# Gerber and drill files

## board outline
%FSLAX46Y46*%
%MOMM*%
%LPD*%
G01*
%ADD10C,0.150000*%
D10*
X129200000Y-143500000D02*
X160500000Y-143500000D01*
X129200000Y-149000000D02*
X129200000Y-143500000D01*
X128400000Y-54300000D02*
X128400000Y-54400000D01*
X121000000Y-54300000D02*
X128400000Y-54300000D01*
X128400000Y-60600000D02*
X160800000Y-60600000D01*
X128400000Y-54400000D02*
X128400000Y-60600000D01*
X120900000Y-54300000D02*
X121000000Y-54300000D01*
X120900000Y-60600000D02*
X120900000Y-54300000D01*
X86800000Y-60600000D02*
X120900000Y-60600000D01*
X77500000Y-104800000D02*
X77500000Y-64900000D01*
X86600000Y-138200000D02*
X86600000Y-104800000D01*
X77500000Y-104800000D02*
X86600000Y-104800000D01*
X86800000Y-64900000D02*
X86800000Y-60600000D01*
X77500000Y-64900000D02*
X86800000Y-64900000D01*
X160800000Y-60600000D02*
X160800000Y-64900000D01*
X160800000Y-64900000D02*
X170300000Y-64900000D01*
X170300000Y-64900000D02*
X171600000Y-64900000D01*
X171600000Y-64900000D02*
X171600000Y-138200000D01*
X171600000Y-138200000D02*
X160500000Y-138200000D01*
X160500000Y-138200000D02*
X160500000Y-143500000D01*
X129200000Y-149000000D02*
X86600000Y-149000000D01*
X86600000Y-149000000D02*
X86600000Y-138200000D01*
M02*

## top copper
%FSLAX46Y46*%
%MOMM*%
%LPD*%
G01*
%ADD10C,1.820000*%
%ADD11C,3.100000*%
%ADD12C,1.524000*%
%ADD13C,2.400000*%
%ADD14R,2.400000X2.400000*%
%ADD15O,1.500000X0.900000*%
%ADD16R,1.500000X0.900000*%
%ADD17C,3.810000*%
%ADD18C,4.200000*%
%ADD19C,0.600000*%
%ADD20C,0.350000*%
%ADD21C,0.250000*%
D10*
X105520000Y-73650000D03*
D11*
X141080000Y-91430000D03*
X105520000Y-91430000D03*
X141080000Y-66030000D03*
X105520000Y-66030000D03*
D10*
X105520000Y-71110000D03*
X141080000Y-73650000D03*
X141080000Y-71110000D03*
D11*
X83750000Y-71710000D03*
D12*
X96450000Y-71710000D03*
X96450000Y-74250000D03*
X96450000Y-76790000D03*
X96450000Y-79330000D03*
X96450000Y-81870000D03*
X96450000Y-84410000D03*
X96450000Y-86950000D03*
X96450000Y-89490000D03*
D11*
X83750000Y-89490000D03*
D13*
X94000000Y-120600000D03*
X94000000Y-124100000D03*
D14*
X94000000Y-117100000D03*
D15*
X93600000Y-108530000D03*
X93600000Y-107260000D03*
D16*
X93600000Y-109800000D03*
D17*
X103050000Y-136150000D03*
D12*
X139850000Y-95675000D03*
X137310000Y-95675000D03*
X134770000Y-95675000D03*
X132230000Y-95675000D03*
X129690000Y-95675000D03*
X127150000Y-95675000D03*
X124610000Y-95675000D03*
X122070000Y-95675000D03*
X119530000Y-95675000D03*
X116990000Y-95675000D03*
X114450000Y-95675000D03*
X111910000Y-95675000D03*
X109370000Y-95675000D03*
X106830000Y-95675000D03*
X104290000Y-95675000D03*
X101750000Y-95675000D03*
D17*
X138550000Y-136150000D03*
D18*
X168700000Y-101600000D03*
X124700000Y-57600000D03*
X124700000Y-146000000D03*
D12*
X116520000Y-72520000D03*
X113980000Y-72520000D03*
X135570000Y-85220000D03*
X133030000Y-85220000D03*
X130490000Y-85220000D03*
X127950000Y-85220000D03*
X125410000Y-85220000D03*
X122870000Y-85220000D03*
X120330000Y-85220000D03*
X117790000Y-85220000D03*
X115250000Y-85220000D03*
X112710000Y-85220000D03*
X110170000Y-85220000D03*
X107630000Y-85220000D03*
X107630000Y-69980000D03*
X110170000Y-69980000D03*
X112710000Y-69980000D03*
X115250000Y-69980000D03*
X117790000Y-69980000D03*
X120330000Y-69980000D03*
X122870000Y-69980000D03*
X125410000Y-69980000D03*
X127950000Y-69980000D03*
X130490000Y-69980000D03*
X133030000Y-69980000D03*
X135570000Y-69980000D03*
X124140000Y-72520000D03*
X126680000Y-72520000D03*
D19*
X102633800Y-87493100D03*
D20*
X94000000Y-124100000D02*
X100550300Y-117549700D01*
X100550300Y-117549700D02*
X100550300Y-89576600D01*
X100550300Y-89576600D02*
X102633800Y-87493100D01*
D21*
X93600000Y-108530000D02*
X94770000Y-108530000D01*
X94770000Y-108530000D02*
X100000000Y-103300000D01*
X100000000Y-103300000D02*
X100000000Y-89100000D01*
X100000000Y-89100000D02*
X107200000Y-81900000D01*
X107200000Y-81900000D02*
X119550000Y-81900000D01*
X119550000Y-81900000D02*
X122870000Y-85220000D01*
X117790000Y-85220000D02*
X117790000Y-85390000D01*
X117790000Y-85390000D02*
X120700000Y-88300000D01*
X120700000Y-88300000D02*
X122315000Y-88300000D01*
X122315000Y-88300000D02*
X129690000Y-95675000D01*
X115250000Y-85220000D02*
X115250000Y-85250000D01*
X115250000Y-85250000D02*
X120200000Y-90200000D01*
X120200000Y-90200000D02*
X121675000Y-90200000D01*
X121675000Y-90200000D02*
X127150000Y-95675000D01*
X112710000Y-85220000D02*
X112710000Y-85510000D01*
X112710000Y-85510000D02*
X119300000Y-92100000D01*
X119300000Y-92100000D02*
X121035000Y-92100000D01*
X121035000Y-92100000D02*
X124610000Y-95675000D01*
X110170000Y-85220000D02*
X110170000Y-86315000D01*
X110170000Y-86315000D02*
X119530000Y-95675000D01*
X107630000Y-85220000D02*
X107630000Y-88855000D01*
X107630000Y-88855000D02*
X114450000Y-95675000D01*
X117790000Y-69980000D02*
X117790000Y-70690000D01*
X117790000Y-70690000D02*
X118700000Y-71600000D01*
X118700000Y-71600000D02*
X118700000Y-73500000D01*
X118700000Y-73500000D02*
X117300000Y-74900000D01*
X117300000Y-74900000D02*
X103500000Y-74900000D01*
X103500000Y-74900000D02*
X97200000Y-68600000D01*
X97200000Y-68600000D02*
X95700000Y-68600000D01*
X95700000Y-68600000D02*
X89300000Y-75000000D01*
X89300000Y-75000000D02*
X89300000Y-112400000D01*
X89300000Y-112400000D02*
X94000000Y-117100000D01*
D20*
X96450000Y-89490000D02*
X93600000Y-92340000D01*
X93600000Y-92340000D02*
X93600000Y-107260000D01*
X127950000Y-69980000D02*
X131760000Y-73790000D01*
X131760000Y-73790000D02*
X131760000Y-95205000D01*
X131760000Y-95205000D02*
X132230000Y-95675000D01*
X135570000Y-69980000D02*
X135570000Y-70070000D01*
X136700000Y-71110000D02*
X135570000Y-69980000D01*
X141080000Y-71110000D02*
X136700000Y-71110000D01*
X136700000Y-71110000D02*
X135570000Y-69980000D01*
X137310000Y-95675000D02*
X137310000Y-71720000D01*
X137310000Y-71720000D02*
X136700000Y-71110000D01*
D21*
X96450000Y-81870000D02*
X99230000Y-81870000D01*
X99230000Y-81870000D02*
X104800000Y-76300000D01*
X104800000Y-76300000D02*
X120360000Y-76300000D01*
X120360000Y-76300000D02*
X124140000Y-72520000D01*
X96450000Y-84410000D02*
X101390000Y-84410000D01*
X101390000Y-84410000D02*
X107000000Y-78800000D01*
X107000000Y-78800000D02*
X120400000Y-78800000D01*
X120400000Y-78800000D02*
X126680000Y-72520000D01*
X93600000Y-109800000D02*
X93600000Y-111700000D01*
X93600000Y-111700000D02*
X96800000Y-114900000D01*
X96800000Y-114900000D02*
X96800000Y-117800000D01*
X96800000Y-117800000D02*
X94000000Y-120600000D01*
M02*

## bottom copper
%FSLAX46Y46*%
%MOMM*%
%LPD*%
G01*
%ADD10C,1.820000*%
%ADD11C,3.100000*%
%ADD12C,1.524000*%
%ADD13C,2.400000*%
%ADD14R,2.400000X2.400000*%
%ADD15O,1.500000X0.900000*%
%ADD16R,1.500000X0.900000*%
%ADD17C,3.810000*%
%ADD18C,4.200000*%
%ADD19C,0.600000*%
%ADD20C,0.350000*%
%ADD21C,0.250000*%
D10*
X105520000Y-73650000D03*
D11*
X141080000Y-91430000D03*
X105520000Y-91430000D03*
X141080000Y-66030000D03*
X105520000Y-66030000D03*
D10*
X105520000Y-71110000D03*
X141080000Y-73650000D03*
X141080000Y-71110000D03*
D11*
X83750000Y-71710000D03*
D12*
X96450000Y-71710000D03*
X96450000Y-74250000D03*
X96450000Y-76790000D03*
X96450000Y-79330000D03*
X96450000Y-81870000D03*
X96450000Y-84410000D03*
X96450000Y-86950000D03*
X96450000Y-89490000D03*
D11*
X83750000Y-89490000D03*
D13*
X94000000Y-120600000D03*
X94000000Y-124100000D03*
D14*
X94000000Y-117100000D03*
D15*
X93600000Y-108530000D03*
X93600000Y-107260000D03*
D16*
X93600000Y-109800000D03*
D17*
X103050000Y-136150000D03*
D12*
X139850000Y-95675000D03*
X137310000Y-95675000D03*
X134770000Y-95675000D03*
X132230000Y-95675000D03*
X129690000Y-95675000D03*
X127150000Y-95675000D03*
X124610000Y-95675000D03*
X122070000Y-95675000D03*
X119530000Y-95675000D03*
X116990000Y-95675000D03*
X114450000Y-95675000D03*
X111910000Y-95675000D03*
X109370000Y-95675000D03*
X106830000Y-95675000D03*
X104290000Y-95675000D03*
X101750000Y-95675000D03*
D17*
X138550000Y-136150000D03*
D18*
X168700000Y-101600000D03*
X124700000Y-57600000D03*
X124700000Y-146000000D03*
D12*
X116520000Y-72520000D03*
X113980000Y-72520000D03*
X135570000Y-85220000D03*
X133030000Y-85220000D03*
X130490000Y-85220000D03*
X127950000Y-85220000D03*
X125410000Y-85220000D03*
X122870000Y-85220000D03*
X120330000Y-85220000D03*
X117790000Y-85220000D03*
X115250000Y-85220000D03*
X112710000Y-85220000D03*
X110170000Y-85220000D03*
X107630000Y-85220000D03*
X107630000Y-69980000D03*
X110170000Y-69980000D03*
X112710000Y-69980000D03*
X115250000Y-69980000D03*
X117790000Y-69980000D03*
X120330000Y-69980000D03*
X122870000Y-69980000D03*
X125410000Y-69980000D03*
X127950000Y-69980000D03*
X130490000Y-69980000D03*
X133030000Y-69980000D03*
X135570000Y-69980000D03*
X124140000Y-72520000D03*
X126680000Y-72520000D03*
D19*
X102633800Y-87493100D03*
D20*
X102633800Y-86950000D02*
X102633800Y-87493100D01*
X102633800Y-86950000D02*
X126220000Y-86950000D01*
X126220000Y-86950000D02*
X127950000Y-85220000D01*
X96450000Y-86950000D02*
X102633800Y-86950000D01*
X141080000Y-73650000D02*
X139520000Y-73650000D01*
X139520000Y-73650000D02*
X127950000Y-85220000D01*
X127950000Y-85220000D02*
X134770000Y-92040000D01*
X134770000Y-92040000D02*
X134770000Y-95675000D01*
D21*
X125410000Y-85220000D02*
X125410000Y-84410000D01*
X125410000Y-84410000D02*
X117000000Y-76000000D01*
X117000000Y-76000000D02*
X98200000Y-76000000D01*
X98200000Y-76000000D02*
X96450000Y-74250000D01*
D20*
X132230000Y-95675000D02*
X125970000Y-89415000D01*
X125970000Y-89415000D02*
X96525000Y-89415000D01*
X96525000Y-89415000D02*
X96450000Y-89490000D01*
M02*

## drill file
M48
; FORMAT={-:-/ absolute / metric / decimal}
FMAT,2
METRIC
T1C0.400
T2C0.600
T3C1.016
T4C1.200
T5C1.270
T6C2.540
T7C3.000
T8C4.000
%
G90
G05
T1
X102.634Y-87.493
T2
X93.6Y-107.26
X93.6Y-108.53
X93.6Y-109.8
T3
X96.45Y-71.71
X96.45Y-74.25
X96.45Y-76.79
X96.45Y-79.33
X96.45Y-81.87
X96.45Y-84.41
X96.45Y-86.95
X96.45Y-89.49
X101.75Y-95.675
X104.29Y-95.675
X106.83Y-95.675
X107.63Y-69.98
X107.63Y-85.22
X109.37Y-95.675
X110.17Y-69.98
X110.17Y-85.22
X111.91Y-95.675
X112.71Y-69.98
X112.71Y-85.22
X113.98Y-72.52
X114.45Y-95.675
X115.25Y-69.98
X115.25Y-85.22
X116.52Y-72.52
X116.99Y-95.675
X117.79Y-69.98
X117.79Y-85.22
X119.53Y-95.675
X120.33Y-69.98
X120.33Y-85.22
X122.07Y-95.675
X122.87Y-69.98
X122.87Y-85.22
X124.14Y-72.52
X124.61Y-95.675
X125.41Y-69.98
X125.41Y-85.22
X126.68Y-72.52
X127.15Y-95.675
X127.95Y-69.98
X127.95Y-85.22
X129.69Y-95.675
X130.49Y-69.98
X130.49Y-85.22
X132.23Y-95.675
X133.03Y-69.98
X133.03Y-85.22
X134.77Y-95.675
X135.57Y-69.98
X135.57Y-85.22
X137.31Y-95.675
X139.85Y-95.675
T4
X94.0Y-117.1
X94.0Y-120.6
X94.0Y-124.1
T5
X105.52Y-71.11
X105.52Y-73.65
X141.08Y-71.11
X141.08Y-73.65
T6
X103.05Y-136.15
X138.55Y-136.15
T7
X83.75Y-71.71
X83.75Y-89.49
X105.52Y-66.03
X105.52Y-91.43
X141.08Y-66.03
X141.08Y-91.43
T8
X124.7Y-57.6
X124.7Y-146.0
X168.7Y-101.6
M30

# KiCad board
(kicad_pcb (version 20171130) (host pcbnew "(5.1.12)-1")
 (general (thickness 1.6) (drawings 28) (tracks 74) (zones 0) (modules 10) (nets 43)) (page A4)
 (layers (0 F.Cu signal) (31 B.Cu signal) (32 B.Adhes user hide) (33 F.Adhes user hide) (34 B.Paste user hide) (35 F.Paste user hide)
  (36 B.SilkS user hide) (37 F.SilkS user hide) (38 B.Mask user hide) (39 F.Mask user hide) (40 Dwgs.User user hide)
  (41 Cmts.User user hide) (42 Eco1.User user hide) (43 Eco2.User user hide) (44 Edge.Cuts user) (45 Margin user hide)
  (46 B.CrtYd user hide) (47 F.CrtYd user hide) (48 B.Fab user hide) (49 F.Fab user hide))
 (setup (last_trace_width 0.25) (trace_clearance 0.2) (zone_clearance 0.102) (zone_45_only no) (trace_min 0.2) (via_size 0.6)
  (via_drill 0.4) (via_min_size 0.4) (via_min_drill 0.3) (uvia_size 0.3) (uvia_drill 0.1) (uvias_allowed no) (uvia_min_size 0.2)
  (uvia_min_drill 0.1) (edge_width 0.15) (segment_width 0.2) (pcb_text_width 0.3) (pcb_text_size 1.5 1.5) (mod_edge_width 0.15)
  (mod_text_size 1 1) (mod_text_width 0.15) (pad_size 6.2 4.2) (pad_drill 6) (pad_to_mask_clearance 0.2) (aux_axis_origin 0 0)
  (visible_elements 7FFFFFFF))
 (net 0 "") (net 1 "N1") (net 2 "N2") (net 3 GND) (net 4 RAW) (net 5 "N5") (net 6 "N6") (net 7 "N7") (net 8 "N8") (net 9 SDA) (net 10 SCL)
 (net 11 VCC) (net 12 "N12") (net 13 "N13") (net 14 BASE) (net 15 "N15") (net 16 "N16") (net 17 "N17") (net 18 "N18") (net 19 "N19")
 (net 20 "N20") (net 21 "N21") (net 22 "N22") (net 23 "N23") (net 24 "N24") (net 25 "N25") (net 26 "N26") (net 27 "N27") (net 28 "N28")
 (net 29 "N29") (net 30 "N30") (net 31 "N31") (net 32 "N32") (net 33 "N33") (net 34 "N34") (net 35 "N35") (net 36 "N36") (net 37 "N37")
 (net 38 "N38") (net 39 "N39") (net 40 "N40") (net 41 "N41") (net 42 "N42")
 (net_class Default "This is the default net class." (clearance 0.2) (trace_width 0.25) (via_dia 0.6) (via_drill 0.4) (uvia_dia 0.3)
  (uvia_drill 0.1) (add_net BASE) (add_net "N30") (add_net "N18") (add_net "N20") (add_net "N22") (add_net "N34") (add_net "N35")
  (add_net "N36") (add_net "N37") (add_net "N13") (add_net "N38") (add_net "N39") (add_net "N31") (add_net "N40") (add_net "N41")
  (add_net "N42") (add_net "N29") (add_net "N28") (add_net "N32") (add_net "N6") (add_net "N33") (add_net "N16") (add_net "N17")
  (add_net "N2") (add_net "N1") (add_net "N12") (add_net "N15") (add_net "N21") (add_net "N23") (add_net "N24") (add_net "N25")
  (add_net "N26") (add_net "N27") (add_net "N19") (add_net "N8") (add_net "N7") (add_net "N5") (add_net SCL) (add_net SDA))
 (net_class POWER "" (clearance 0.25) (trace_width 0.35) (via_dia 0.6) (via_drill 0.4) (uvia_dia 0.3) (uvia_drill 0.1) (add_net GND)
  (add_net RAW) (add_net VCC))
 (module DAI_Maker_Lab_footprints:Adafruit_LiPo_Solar (layer F.Cu) (at 123.3 80)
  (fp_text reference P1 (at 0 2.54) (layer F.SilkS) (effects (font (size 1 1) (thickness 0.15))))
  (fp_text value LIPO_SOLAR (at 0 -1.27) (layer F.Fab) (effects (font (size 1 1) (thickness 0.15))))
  (pad 2 thru_hole circle (at -17.78 -6.35) (size 1.82 1.82) (drill 1.27) (layers *.Cu *.Mask F.SilkS) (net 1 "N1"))
  (pad "" thru_hole circle (at 17.78 11.43) (size 3.1 3.1) (drill 3) (layers *.Cu *.Mask F.SilkS))
  (pad "" thru_hole circle (at -17.78 11.43) (size 3.1 3.1) (drill 3) (layers *.Cu *.Mask F.SilkS))
  (pad "" thru_hole circle (at 17.78 -13.97) (size 3.1 3.1) (drill 3) (layers *.Cu *.Mask F.SilkS))
  (pad "" thru_hole circle (at -17.78 -13.97) (size 3.1 3.1) (drill 3) (layers *.Cu *.Mask F.SilkS))
  (pad 1 thru_hole circle (at -17.78 -8.89) (size 1.82 1.82) (drill 1.27) (layers *.Cu *.Mask F.SilkS) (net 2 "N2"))
  (pad 4 thru_hole circle (at 17.78 -6.35) (size 1.82 1.82) (drill 1.27) (layers *.Cu *.Mask F.SilkS) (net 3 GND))
  (pad 3 thru_hole circle (at 17.78 -8.89) (size 1.82 1.82) (drill 1.27) (layers *.Cu *.Mask F.SilkS) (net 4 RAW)))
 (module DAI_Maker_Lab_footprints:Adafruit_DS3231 (layer F.Cu) (at 90.1 80.6 90)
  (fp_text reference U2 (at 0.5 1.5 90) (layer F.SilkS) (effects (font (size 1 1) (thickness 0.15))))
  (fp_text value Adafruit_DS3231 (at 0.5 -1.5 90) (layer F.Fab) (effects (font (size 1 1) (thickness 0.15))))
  (pad "" thru_hole circle (at 8.89 -6.35 90) (size 3.1 3.1) (drill 3) (layers *.Cu *.Mask F.SilkS))
  (pad 8 thru_hole circle (at 8.89 6.35 90) (size 1.524 1.524) (drill 1.016) (layers *.Cu *.Mask F.SilkS) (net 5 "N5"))
  (pad 7 thru_hole circle (at 6.35 6.35 90) (size 1.524 1.524) (drill 1.016) (layers *.Cu *.Mask F.SilkS) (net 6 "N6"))
  (pad 6 thru_hole circle (at 3.81 6.35 90) (size 1.524 1.524) (drill 1.016) (layers *.Cu *.Mask F.SilkS) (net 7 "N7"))
  (pad 5 thru_hole circle (at 1.27 6.35 90) (size 1.524 1.524) (drill 1.016) (layers *.Cu *.Mask F.SilkS) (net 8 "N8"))
  (pad 4 thru_hole circle (at -1.27 6.35 90) (size 1.524 1.524) (drill 1.016) (layers *.Cu *.Mask F.SilkS) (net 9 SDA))
  (pad 3 thru_hole circle (at -3.81 6.35 90) (size 1.524 1.524) (drill 1.016) (layers *.Cu *.Mask F.SilkS) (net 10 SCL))
  (pad 2 thru_hole circle (at -6.35 6.35 90) (size 1.524 1.524) (drill 1.016) (layers *.Cu *.Mask F.SilkS) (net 3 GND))
  (pad 1 thru_hole circle (at -8.89 6.35 90) (size 1.524 1.524) (drill 1.016) (layers *.Cu *.Mask F.SilkS) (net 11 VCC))
  (pad "" thru_hole circle (at -8.89 -6.35 90) (size 3.1 3.1) (drill 3) (layers *.Cu *.Mask F.SilkS)))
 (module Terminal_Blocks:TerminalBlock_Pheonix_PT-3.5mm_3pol (layer F.Cu) (at 94 117.1 270)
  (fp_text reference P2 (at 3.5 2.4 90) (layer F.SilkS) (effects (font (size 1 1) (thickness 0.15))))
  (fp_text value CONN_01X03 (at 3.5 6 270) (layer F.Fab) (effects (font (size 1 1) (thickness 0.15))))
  (pad 2 thru_hole circle (at 3.5 0 270) (size 2.4 2.4) (drill 1.2) (layers *.Cu *.Mask) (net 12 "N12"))
  (pad 3 thru_hole circle (at 7 0 270) (size 2.4 2.4) (drill 1.2) (layers *.Cu *.Mask) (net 3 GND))
  (pad 1 thru_hole rect (at 0 0 270) (size 2.4 2.4) (drill 1.2) (layers *.Cu *.Mask) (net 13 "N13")))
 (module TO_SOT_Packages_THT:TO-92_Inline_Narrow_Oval (layer F.Cu) (at 93.6 109.8 90)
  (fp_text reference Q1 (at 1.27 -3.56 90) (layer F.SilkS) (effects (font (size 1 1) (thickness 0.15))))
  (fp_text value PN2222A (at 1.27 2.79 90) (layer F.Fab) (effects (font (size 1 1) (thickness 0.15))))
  (pad 2 thru_hole oval (at 1.27 0 270) (size 0.9 1.5) (drill 0.6) (layers *.Cu *.Mask) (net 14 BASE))
  (pad 3 thru_hole oval (at 2.54 0 270) (size 0.9 1.5) (drill 0.6) (layers *.Cu *.Mask) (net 11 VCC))
  (pad 1 thru_hole rect (at 0 0 270) (size 0.9 1.5) (drill 0.6) (layers *.Cu *.Mask) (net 12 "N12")))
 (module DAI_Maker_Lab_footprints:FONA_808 (layer F.Cu) (at 120.8 117.9 180)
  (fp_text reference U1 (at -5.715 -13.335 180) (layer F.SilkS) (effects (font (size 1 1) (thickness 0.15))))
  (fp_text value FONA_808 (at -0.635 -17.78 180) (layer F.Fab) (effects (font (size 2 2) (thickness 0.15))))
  (pad 18 thru_hole circle (at 17.75 -18.25 180) (size 3.81 3.81) (drill 2.54) (layers *.Cu *.Mask F.SilkS))
  (pad 1 thru_hole circle (at -19.05 22.225 180) (size 1.524 1.524) (drill 1.016) (layers *.Cu *.Mask F.SilkS) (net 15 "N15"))
  (pad 2 thru_hole circle (at -16.51 22.225 180) (size 1.524 1.524) (drill 1.016) (layers *.Cu *.Mask F.SilkS) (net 4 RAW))
  (pad 3 thru_hole circle (at -13.97 22.225 180) (size 1.524 1.524) (drill 1.016) (layers *.Cu *.Mask F.SilkS) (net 3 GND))
  (pad 4 thru_hole circle (at -11.43 22.225 180) (size 1.524 1.524) (drill 1.016) (layers *.Cu *.Mask F.SilkS) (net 11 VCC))
  (pad 5 thru_hole circle (at -8.89 22.225 180) (size 1.524 1.524) (drill 1.016) (layers *.Cu *.Mask F.SilkS) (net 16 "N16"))
  (pad 6 thru_hole circle (at -6.35 22.225 180) (size 1.524 1.524) (drill 1.016) (layers *.Cu *.Mask F.SilkS) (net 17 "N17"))
  (pad 7 thru_hole circle (at -3.81 22.225 180) (size 1.524 1.524) (drill 1.016) (layers *.Cu *.Mask F.SilkS) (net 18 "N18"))
  (pad 8 thru_hole circle (at -1.27 22.225 180) (size 1.524 1.524) (drill 1.016) (layers *.Cu *.Mask F.SilkS) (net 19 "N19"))
  (pad 9 thru_hole circle (at 1.27 22.225 180) (size 1.524 1.524) (drill 1.016) (layers *.Cu *.Mask F.SilkS) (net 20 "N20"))
  (pad 10 thru_hole circle (at 3.81 22.225 180) (size 1.524 1.524) (drill 1.016) (layers *.Cu *.Mask F.SilkS) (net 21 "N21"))
  (pad 11 thru_hole circle (at 6.35 22.225 180) (size 1.524 1.524) (drill 1.016) (layers *.Cu *.Mask F.SilkS) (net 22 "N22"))
  (pad 12 thru_hole circle (at 8.89 22.225 180) (size 1.524 1.524) (drill 1.016) (layers *.Cu *.Mask F.SilkS) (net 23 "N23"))
  (pad 13 thru_hole circle (at 11.43 22.225 180) (size 1.524 1.524) (drill 1.016) (layers *.Cu *.Mask F.SilkS) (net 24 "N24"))
  (pad 14 thru_hole circle (at 13.97 22.225 180) (size 1.524 1.524) (drill 1.016) (layers *.Cu *.Mask F.SilkS) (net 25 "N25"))
  (pad 15 thru_hole circle (at 16.51 22.225 180) (size 1.524 1.524) (drill 1.016) (layers *.Cu *.Mask F.SilkS) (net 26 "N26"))
  (pad 16 thru_hole circle (at 19.05 22.225 180) (size 1.524 1.524) (drill 1.016) (layers *.Cu *.Mask F.SilkS) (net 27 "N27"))
  (pad 17 thru_hole circle (at -17.75 -18.25 180) (size 3.81 3.81) (drill 2.54) (layers *.Cu *.Mask F.SilkS)))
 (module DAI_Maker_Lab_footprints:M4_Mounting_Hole (layer F.Cu) (at 168.7 101.6)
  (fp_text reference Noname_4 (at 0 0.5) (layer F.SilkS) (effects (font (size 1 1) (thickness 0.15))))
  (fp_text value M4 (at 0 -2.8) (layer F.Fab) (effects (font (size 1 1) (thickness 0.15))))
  (pad "" thru_hole circle (at 0 0) (size 4.2 4.2) (drill 4) (layers *.Cu *.Mask F.SilkS)))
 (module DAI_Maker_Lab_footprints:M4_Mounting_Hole (layer F.Cu) (at 124.7 57.6)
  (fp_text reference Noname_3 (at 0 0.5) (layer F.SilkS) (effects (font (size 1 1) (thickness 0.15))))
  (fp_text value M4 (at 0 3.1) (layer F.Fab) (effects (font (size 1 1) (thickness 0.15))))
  (pad "" thru_hole circle (at 0 0) (size 4.2 4.2) (drill 4) (layers *.Cu *.Mask F.SilkS)))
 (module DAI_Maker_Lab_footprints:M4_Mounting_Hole (layer F.Cu) (at 124.7 146)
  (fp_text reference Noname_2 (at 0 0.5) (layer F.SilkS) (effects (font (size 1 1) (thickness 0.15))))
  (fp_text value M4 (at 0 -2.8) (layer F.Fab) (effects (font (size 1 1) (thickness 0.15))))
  (pad "" thru_hole circle (at 0 0) (size 4.2 4.2) (drill 4) (layers *.Cu *.Mask F.SilkS)))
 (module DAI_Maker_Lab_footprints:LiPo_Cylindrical (layer F.Cu) (at 157.1 100.3 90)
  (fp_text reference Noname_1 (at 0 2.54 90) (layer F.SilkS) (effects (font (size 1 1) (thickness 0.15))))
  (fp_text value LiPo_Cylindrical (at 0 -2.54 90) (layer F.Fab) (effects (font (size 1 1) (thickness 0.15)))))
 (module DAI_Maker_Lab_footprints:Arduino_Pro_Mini (layer B.Cu) (at 121.6 77.6 180)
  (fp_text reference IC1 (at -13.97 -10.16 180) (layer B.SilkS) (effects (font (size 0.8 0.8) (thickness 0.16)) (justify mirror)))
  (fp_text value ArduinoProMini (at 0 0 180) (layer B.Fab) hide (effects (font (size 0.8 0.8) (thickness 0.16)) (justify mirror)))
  (pad 28 thru_hole circle (at 5.08 5.08 180) (size 1.524 1.524) (drill 1.016) (layers *.Cu *.Mask B.SilkS) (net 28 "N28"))
  (pad 27 thru_hole circle (at 7.62 5.08 180) (size 1.524 1.524) (drill 1.016) (layers *.Cu *.Mask B.SilkS) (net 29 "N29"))
  (pad 1 thru_hole circle (at -13.97 -7.62 180) (size 1.524 1.524) (drill 1.016) (layers *.Cu *.Mask B.SilkS) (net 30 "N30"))
  (pad 2 thru_hole circle (at -11.43 -7.62 180) (size 1.524 1.524) (drill 1.016) (layers *.Cu *.Mask B.SilkS) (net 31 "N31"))
  (pad 3 thru_hole circle (at -8.89 -7.62 180) (size 1.524 1.524) (drill 1.016) (layers *.Cu *.Mask B.SilkS) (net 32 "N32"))
  (pad 4 thru_hole circle (at -6.35 -7.62 180) (size 1.524 1.524) (drill 1.016) (layers *.Cu *.Mask B.SilkS) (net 3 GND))
  (pad 5 thru_hole circle (at -3.81 -7.62 180) (size 1.524 1.524) (drill 1.016) (layers *.Cu *.Mask B.SilkS) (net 6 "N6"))
  (pad 6 thru_hole circle (at -1.27 -7.62 180) (size 1.524 1.524) (drill 1.016) (layers *.Cu *.Mask B.SilkS) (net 14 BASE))
  (pad 7 thru_hole circle (at 1.27 -7.62 180) (size 1.524 1.524) (drill 1.016) (layers *.Cu *.Mask B.SilkS) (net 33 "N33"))
  (pad 8 thru_hole circle (at 3.81 -7.62 180) (size 1.524 1.524) (drill 1.016) (layers *.Cu *.Mask B.SilkS) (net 16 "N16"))
  (pad 9 thru_hole circle (at 6.35 -7.62 180) (size 1.524 1.524) (drill 1.016) (layers *.Cu *.Mask B.SilkS) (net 17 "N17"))
  (pad 10 thru_hole circle (at 8.89 -7.62 180) (size 1.524 1.524) (drill 1.016) (layers *.Cu *.Mask B.SilkS) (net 18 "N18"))
  (pad 11 thru_hole circle (at 11.43 -7.62 180) (size 1.524 1.524) (drill 1.016) (layers *.Cu *.Mask B.SilkS) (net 20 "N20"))
  (pad 12 thru_hole circle (at 13.97 -7.62 180) (size 1.524 1.524) (drill 1.016) (layers *.Cu *.Mask B.SilkS) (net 22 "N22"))
  (pad 13 thru_hole circle (at 13.97 7.62 180) (size 1.524 1.524) (drill 1.016) (layers *.Cu *.Mask B.SilkS) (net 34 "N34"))
  (pad 14 thru_hole circle (at 11.43 7.62 180) (size 1.524 1.524) (drill 1.016) (layers *.Cu *.Mask B.SilkS) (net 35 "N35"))
  (pad 15 thru_hole circle (at 8.89 7.62 180) (size 1.524 1.524) (drill 1.016) (layers *.Cu *.Mask B.SilkS) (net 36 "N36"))
  (pad 16 thru_hole circle (at 6.35 7.62 180) (size 1.524 1.524) (drill 1.016) (layers *.Cu *.Mask B.SilkS) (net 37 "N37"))
  (pad 17 thru_hole circle (at 3.81 7.62 180) (size 1.524 1.524) (drill 1.016) (layers *.Cu *.Mask B.SilkS) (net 13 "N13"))
  (pad 18 thru_hole circle (at 1.27 7.62 180) (size 1.524 1.524) (drill 1.016) (layers *.Cu *.Mask B.SilkS) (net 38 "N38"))
  (pad 19 thru_hole circle (at -1.27 7.62 180) (size 1.524 1.524) (drill 1.016) (layers *.Cu *.Mask B.SilkS) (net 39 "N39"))
  (pad 20 thru_hole circle (at -3.81 7.62 180) (size 1.524 1.524) (drill 1.016) (layers *.Cu *.Mask B.SilkS) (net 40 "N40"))
  (pad 21 thru_hole circle (at -6.35 7.62 180) (size 1.524 1.524) (drill 1.016) (layers *.Cu *.Mask B.SilkS) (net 11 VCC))
  (pad 22 thru_hole circle (at -8.89 7.62 180) (size 1.524 1.524) (drill 1.016) (layers *.Cu *.Mask B.SilkS) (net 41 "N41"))
  (pad 23 thru_hole circle (at -11.43 7.62 180) (size 1.524 1.524) (drill 1.016) (layers *.Cu *.Mask B.SilkS) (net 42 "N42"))
  (pad 24 thru_hole circle (at -13.97 7.62 180) (size 1.524 1.524) (drill 1.016) (layers *.Cu *.Mask B.SilkS) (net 4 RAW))
  (pad 25 thru_hole circle (at -2.54 5.08 180) (size 1.524 1.524) (drill 1.016) (layers *.Cu *.Mask B.SilkS) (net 9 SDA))
  (pad 26 thru_hole circle (at -5.08 5.08 180) (size 1.524 1.524) (drill 1.016) (layers *.Cu *.Mask B.SilkS) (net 10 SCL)))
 (gr_line (start 129.2 143.5) (end 160.5 143.5) (angle 90) (layer Edge.Cuts) (width 0.15))
 (gr_line (start 129.2 149) (end 129.2 143.5) (angle 90) (layer Edge.Cuts) (width 0.15))
 (gr_line (start 128.4 54.3) (end 128.4 54.4) (angle 90) (layer Edge.Cuts) (width 0.15))
 (gr_line (start 121 54.3) (end 128.4 54.3) (angle 90) (layer Edge.Cuts) (width 0.15))
 (gr_line (start 128.4 60.6) (end 160.8 60.6) (angle 90) (layer Edge.Cuts) (width 0.15))
 (gr_line (start 128.4 54.4) (end 128.4 60.6) (angle 90) (layer Edge.Cuts) (width 0.15))
 (gr_line (start 120.9 54.3) (end 121 54.3) (angle 90) (layer Edge.Cuts) (width 0.15))
 (gr_line (start 120.9 60.6) (end 120.9 54.3) (angle 90) (layer Edge.Cuts) (width 0.15))
 (gr_line (start 86.8 60.6) (end 120.9 60.6) (angle 90) (layer Edge.Cuts) (width 0.15))
 (gr_line (start 77.5 104.8) (end 77.5 64.9) (angle 90) (layer Edge.Cuts) (width 0.15))
 (gr_line (start 86.6 138.2) (end 86.6 104.8) (angle 90) (layer Edge.Cuts) (width 0.15))
 (gr_line (start 77.5 104.8) (end 86.6 104.8) (angle 90) (layer Edge.Cuts) (width 0.15))
 (gr_line (start 86.8 64.9) (end 86.8 60.6) (angle 90) (layer Edge.Cuts) (width 0.15))
 (gr_line (start 77.5 64.9) (end 86.8 64.9) (angle 90) (layer Edge.Cuts) (width 0.15))
 (gr_line (start 160.8 60.6) (end 160.8 64.9) (angle 90) (layer Edge.Cuts) (width 0.15))
 (gr_line (start 160.8 64.9) (end 170.3 64.9) (angle 90) (layer Edge.Cuts) (width 0.15))
 (gr_line (start 170.3 64.9) (end 171.6 64.9) (angle 90) (layer Edge.Cuts) (width 0.15))
 (gr_line (start 171.6 64.9) (end 171.6 138.2) (angle 90) (layer Edge.Cuts) (width 0.15))
 (gr_line (start 171.6 138.2) (end 160.5 138.2) (angle 90) (layer Edge.Cuts) (width 0.15))
 (gr_line (start 160.5 138.2) (end 160.5 143.5) (angle 90) (layer Edge.Cuts) (width 0.15))
 (gr_line (start 129.2 149) (end 86.6 149) (angle 90) (layer Edge.Cuts) (width 0.15))
 (gr_line (start 86.6 149) (end 86.6 138.2) (angle 90) (layer Edge.Cuts) (width 0.15))
 (segment (start 94 124.1) (end 100.5503 117.5497) (width 0.35) (layer F.Cu) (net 3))
 (segment (start 100.5503 117.5497) (end 100.5503 89.5766) (width 0.35) (layer F.Cu) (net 3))
 (segment (start 100.5503 89.5766) (end 102.6338 87.4931) (width 0.35) (layer F.Cu) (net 3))
 (segment (start 102.6338 86.95) (end 102.6338 87.4931) (width 0.35) (layer B.Cu) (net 3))
 (segment (start 102.6338 86.95) (end 126.22 86.95) (width 0.35) (layer B.Cu) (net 3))
 (segment (start 126.22 86.95) (end 127.95 85.22) (width 0.35) (layer B.Cu) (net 3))
 (segment (start 96.45 86.95) (end 102.6338 86.95) (width 0.35) (layer B.Cu) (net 3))
 (segment (start 141.08 73.65) (end 139.52 73.65) (width 0.35) (layer B.Cu) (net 3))
 (segment (start 139.52 73.65) (end 127.95 85.22) (width 0.35) (layer B.Cu) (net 3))
 (segment (start 127.95 85.22) (end 134.77 92.04) (width 0.35) (layer B.Cu) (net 3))
 (segment (start 134.77 92.04) (end 134.77 95.675) (width 0.35) (layer B.Cu) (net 3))
 (via (at 102.6338 87.4931) (size 0.6) (layers F.Cu B.Cu) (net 3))
 (segment (start 125.41 85.22) (end 125.41 84.41) (width 0.25) (layer B.Cu) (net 6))
 (segment (start 125.41 84.41) (end 117 76) (width 0.25) (layer B.Cu) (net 6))
 (segment (start 117 76) (end 98.2 76) (width 0.25) (layer B.Cu) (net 6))
 (segment (start 98.2 76) (end 96.45 74.25) (width 0.25) (layer B.Cu) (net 6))
 (segment (start 93.6 108.53) (end 94.77 108.53) (width 0.25) (layer F.Cu) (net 14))
 (segment (start 94.77 108.53) (end 100 103.3) (width 0.25) (layer F.Cu) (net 14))
 (segment (start 100 103.3) (end 100 89.1) (width 0.25) (layer F.Cu) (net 14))
 (segment (start 100 89.1) (end 107.2 81.9) (width 0.25) (layer F.Cu) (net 14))
 (segment (start 107.2 81.9) (end 119.55 81.9) (width 0.25) (layer F.Cu) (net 14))
 (segment (start 119.55 81.9) (end 122.87 85.22) (width 0.25) (layer F.Cu) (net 14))
 (segment (start 117.79 85.22) (end 117.79 85.39) (width 0.25) (layer F.Cu) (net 16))
 (segment (start 117.79 85.39) (end 120.7 88.3) (width 0.25) (layer F.Cu) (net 16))
 (segment (start 120.7 88.3) (end 122.315 88.3) (width 0.25) (layer F.Cu) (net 16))
 (segment (start 122.315 88.3) (end 129.69 95.675) (width 0.25) (layer F.Cu) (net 16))
 (segment (start 115.25 85.22) (end 115.25 85.25) (width 0.25) (layer F.Cu) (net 17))
 (segment (start 115.25 85.25) (end 120.2 90.2) (width 0.25) (layer F.Cu) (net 17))
 (segment (start 120.2 90.2) (end 121.675 90.2) (width 0.25) (layer F.Cu) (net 17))
 (segment (start 121.675 90.2) (end 127.15 95.675) (width 0.25) (layer F.Cu) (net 17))
 (segment (start 112.71 85.22) (end 112.71 85.51) (width 0.25) (layer F.Cu) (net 18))
 (segment (start 112.71 85.51) (end 119.3 92.1) (width 0.25) (layer F.Cu) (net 18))
 (segment (start 119.3 92.1) (end 121.035 92.1) (width 0.25) (layer F.Cu) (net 18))
 (segment (start 121.035 92.1) (end 124.61 95.675) (width 0.25) (layer F.Cu) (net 18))
 (segment (start 110.17 85.22) (end 110.17 86.315) (width 0.25) (layer F.Cu) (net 20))
 (segment (start 110.17 86.315) (end 119.53 95.675) (width 0.25) (layer F.Cu) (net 20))
 (segment (start 107.63 85.22) (end 107.63 88.855) (width 0.25) (layer F.Cu) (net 22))
 (segment (start 107.63 88.855) (end 114.45 95.675) (width 0.25) (layer F.Cu) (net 22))
 (segment (start 117.79 69.98) (end 117.79 70.69) (width 0.25) (layer F.Cu) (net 13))
 (segment (start 117.79 70.69) (end 118.7 71.6) (width 0.25) (layer F.Cu) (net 13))
 (segment (start 118.7 71.6) (end 118.7 73.5) (width 0.25) (layer F.Cu) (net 13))
 (segment (start 118.7 73.5) (end 117.3 74.9) (width 0.25) (layer F.Cu) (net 13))
 (segment (start 117.3 74.9) (end 103.5 74.9) (width 0.25) (layer F.Cu) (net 13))
 (segment (start 103.5 74.9) (end 97.2 68.6) (width 0.25) (layer F.Cu) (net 13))
 (segment (start 97.2 68.6) (end 95.7 68.6) (width 0.25) (layer F.Cu) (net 13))
 (segment (start 95.7 68.6) (end 89.3 75) (width 0.25) (layer F.Cu) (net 13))
 (segment (start 89.3 75) (end 89.3 112.4) (width 0.25) (layer F.Cu) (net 13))
 (segment (start 89.3 112.4) (end 94 117.1) (width 0.25) (layer F.Cu) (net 13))
 (segment (start 132.23 95.675) (end 125.97 89.415) (width 0.35) (layer B.Cu) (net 11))
 (segment (start 125.97 89.415) (end 96.525 89.415) (width 0.35) (layer B.Cu) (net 11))
 (segment (start 96.525 89.415) (end 96.45 89.49) (width 0.35) (layer B.Cu) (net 11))
 (segment (start 96.45 89.49) (end 93.6 92.34) (width 0.35) (layer F.Cu) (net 11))
 (segment (start 93.6 92.34) (end 93.6 107.26) (width 0.35) (layer F.Cu) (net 11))
 (segment (start 127.95 69.98) (end 131.76 73.79) (width 0.35) (layer F.Cu) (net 11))
 (segment (start 131.76 73.79) (end 131.76 95.205) (width 0.35) (layer F.Cu) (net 11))
 (segment (start 131.76 95.205) (end 132.23 95.675) (width 0.35) (layer F.Cu) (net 11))
 (segment (start 135.57 69.98) (end 135.57 70.07) (width 0.35) (layer F.Cu) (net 4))
 (segment (start 136.7 71.11) (end 135.57 69.98) (width 0.35) (layer F.Cu) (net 4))
 (segment (start 141.08 71.11) (end 136.7 71.11) (width 0.35) (layer F.Cu) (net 4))
 (segment (start 136.7 71.11) (end 135.57 69.98) (width 0.35) (layer F.Cu) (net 4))
 (segment (start 137.31 95.675) (end 137.31 71.72) (width 0.35) (layer F.Cu) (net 4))
 (segment (start 137.31 71.72) (end 136.7 71.11) (width 0.35) (layer F.Cu) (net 4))
 (segment (start 96.45 81.87) (end 99.23 81.87) (width 0.25) (layer F.Cu) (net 9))
 (segment (start 99.23 81.87) (end 104.8 76.3) (width 0.25) (layer F.Cu) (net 9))
 (segment (start 104.8 76.3) (end 120.36 76.3) (width 0.25) (layer F.Cu) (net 9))
 (segment (start 120.36 76.3) (end 124.14 72.52) (width 0.25) (layer F.Cu) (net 9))
 (segment (start 96.45 84.41) (end 101.39 84.41) (width 0.25) (layer F.Cu) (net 10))
 (segment (start 101.39 84.41) (end 107 78.8) (width 0.25) (layer F.Cu) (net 10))
 (segment (start 107 78.8) (end 120.4 78.8) (width 0.25) (layer F.Cu) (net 10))
 (segment (start 120.4 78.8) (end 126.68 72.52) (width 0.25) (layer F.Cu) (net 10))
 (segment (start 93.6 109.8) (end 93.6 111.7) (width 0.25) (layer F.Cu) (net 12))
 (segment (start 93.6 111.7) (end 96.8 114.9) (width 0.25) (layer F.Cu) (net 12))
 (segment (start 96.8 114.9) (end 96.8 117.8) (width 0.25) (layer F.Cu) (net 12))
 (segment (start 96.8 117.8) (end 94 120.6) (width 0.25) (layer F.Cu) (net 12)))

